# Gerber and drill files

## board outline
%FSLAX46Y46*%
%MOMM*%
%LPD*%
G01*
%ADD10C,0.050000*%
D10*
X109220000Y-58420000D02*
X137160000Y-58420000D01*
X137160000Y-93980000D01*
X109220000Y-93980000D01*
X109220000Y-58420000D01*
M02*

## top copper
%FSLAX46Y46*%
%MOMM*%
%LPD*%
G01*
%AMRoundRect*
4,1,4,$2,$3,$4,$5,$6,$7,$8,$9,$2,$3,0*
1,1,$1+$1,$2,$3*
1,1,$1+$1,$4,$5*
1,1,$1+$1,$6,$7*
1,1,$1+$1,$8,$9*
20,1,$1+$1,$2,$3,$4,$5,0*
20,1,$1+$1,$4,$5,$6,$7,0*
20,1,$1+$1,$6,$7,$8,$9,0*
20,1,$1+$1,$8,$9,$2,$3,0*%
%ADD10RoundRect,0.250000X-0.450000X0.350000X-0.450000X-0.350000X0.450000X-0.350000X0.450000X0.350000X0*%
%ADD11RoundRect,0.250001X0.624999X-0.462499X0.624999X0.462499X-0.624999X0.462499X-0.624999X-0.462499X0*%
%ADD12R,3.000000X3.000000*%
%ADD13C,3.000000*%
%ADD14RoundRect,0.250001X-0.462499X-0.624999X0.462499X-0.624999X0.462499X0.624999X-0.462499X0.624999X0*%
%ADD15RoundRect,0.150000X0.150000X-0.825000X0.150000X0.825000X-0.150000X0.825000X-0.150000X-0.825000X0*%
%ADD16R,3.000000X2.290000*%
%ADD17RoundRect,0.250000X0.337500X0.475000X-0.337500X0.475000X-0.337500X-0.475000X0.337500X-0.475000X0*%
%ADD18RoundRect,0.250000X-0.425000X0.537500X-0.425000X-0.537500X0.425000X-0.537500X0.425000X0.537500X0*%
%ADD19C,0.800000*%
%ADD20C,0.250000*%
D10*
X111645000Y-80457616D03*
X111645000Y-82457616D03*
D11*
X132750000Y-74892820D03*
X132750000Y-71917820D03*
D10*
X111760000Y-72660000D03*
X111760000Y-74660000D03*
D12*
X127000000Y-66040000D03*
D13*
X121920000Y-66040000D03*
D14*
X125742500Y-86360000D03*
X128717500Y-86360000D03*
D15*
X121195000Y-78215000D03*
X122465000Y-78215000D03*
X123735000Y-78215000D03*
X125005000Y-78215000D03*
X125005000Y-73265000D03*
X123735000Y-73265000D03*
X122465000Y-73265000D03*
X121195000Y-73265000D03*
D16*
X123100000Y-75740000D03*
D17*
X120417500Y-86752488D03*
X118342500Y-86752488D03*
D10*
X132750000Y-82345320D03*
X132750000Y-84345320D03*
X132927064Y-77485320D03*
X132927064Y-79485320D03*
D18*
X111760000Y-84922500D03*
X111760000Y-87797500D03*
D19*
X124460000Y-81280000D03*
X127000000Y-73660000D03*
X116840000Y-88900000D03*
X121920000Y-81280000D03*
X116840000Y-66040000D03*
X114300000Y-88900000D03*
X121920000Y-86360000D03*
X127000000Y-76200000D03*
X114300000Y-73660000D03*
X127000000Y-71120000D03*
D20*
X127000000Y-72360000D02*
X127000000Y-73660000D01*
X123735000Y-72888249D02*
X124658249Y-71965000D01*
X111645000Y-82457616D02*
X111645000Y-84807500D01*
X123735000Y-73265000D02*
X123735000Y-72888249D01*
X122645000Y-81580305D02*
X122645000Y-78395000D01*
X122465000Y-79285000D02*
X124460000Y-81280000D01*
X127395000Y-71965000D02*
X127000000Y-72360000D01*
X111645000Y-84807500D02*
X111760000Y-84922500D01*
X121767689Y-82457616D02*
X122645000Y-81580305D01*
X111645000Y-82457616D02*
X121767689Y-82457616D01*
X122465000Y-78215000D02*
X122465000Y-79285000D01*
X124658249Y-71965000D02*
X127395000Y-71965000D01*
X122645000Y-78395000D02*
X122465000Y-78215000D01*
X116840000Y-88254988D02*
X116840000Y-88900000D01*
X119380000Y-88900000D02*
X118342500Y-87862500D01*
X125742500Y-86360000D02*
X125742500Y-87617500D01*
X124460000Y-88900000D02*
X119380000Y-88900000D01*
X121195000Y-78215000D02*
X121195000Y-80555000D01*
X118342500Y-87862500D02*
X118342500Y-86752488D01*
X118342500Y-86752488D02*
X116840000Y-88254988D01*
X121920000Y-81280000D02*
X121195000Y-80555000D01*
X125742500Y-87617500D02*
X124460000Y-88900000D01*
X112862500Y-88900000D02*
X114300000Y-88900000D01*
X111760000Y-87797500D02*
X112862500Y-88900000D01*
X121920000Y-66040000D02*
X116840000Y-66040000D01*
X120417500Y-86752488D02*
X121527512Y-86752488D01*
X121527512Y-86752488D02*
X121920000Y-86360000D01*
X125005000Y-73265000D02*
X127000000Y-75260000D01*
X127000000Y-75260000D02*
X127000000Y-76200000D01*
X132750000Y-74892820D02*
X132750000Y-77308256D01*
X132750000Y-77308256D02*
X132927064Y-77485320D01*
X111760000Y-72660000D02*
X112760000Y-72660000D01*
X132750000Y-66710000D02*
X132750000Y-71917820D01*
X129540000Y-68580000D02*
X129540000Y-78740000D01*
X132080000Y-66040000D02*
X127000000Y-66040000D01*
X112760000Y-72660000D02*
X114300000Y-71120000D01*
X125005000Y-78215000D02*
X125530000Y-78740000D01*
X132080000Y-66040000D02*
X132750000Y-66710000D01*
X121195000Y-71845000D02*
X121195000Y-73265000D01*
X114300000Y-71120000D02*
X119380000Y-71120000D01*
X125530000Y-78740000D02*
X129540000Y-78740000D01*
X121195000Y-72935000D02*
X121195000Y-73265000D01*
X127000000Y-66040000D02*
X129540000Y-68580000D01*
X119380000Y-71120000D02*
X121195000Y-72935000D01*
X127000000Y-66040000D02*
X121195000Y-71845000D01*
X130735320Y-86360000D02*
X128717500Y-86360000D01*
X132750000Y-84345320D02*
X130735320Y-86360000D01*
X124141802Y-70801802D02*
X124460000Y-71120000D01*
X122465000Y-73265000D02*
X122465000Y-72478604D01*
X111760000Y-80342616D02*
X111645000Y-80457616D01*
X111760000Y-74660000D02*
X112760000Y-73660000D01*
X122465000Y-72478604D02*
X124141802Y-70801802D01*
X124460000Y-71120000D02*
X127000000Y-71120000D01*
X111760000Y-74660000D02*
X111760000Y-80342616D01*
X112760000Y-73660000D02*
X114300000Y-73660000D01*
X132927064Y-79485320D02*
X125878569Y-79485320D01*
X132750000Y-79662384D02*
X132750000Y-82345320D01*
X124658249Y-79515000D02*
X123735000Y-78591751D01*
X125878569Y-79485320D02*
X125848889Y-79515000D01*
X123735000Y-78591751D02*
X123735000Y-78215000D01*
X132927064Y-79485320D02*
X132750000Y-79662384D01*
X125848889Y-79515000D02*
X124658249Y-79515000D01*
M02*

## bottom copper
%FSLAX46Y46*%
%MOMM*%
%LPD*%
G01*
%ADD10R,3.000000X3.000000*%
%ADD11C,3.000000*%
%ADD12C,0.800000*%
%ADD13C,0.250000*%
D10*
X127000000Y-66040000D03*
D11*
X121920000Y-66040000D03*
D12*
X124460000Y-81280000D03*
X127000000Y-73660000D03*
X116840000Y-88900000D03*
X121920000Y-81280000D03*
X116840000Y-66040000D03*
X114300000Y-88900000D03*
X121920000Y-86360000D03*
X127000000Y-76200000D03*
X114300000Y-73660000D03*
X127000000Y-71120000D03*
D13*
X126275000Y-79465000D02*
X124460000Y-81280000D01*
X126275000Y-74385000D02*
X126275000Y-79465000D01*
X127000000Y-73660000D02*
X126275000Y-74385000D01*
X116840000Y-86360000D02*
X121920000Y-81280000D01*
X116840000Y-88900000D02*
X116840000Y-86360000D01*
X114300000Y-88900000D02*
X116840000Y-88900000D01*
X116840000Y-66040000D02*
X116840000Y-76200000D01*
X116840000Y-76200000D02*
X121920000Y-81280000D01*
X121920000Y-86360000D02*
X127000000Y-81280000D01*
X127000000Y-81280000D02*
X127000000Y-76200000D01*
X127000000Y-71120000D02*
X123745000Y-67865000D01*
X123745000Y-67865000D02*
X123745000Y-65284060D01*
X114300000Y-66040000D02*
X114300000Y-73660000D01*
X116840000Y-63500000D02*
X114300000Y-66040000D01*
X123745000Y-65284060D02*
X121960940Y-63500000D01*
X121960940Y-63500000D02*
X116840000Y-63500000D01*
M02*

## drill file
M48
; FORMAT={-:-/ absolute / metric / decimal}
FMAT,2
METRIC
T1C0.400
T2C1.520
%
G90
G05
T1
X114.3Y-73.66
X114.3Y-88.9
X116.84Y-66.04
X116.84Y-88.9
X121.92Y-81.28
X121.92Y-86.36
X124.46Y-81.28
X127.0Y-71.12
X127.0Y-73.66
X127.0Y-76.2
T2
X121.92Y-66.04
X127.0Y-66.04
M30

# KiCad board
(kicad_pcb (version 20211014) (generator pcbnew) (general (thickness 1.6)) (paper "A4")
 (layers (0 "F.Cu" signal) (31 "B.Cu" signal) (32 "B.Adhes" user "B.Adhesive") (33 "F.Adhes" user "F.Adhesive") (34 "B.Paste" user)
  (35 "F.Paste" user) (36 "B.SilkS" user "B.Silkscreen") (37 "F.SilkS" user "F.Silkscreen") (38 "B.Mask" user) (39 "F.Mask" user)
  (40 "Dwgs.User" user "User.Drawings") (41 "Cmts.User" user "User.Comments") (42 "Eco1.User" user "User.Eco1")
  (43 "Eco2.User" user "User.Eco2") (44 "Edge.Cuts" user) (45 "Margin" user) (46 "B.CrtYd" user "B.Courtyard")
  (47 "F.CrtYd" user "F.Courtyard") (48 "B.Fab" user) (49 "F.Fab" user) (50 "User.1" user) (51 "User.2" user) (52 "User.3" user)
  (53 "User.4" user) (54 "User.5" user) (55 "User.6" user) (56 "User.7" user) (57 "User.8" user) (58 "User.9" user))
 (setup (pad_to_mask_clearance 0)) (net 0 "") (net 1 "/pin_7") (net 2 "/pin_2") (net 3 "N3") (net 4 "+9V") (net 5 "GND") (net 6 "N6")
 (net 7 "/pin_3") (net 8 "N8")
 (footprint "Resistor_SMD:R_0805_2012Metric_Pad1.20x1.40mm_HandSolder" (layer "F.Cu") (at 111.645 81.457616 -90)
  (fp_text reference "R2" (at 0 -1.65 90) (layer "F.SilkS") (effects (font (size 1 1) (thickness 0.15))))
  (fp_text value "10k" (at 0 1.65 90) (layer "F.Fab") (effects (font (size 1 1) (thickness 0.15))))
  (pad "1" smd roundrect (at -1 0 270) (size 1.2 1.4) (layers "F.Cu" "F.Paste" "F.Mask") (roundrect_rratio 0.208333) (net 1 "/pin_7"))
  (pad "2" smd roundrect (at 1 0 270) (size 1.2 1.4) (layers "F.Cu" "F.Paste" "F.Mask") (roundrect_rratio 0.208333) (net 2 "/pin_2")))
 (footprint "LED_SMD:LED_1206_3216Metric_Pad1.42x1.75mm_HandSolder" (layer "F.Cu") (at 132.75 73.40532 90)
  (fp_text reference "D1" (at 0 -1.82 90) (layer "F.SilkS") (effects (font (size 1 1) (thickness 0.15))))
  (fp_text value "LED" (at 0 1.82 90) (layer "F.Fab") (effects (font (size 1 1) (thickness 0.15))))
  (pad "1" smd roundrect (at -1.4875 0 90) (size 1.425 1.75) (layers "F.Cu" "F.Paste" "F.Mask") (roundrect_rratio 0.175439) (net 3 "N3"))
  (pad "2" smd roundrect (at 1.4875 0 90) (size 1.425 1.75) (layers "F.Cu" "F.Paste" "F.Mask") (roundrect_rratio 0.175439) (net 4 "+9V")))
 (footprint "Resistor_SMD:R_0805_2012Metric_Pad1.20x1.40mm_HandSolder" (layer "F.Cu") (at 111.76 73.66 -90)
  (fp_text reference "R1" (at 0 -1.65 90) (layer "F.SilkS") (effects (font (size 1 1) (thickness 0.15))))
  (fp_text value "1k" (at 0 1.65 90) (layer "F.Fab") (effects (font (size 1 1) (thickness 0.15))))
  (pad "1" smd roundrect (at -1 0 270) (size 1.2 1.4) (layers "F.Cu" "F.Paste" "F.Mask") (roundrect_rratio 0.208333) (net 4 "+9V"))
  (pad "2" smd roundrect (at 1 0 270) (size 1.2 1.4) (layers "F.Cu" "F.Paste" "F.Mask") (roundrect_rratio 0.208333) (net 1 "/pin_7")))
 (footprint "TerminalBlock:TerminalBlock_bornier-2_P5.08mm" (layer "F.Cu") (at 127 66.04 180)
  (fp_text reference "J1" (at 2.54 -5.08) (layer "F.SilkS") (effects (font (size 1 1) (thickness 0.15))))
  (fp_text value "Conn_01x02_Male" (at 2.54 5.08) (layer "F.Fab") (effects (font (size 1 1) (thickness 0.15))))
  (pad "1" thru_hole rect (at 0 0 180) (size 3 3) (drill 1.52) (layers *.Cu *.Mask) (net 4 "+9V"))
  (pad "2" thru_hole circle (at 5.08 0 180) (size 3 3) (drill 1.52) (layers *.Cu *.Mask) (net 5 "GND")))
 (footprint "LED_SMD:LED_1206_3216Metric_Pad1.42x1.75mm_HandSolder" (layer "F.Cu") (at 127.23 86.36)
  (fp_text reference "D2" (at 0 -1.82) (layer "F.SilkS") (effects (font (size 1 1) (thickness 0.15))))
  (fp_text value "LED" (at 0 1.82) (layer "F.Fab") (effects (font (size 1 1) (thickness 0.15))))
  (pad "1" smd roundrect (at -1.4875 0) (size 1.425 1.75) (layers "F.Cu" "F.Paste" "F.Mask") (roundrect_rratio 0.175439) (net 5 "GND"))
  (pad "2" smd roundrect (at 1.4875 0) (size 1.425 1.75) (layers "F.Cu" "F.Paste" "F.Mask") (roundrect_rratio 0.175439) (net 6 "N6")))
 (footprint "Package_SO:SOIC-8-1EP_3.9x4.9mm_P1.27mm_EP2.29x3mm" (layer "F.Cu") (at 123.1 75.74 90)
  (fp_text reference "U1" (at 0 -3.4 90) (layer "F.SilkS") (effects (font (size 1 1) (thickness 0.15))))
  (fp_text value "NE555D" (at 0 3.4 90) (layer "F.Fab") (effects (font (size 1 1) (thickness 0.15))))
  (pad "" smd roundrect (at 0.57 -0.75 90) (size 0.92 1.21) (layers "F.Paste") (roundrect_rratio 0.25))
  (pad "" smd roundrect (at 0.57 0.75 90) (size 0.92 1.21) (layers "F.Paste") (roundrect_rratio 0.25))
  (pad "" smd roundrect (at -0.57 0.75 90) (size 0.92 1.21) (layers "F.Paste") (roundrect_rratio 0.25))
  (pad "" smd roundrect (at -0.57 -0.75 90) (size 0.92 1.21) (layers "F.Paste") (roundrect_rratio 0.25))
  (pad "1" smd roundrect (at -2.475 -1.905 90) (size 1.95 0.6) (layers "F.Cu" "F.Paste" "F.Mask") (roundrect_rratio 0.25) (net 5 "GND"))
  (pad "2" smd roundrect (at -2.475 -0.635 90) (size 1.95 0.6) (layers "F.Cu" "F.Paste" "F.Mask") (roundrect_rratio 0.25) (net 2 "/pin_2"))
  (pad "3" smd roundrect (at -2.475 0.635 90) (size 1.95 0.6) (layers "F.Cu" "F.Paste" "F.Mask") (roundrect_rratio 0.25) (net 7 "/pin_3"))
  (pad "4" smd roundrect (at -2.475 1.905 90) (size 1.95 0.6) (layers "F.Cu" "F.Paste" "F.Mask") (roundrect_rratio 0.25) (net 4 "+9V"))
  (pad "5" smd roundrect (at 2.475 1.905 90) (size 1.95 0.6) (layers "F.Cu" "F.Paste" "F.Mask") (roundrect_rratio 0.25) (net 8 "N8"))
  (pad "6" smd roundrect (at 2.475 0.635 90) (size 1.95 0.6) (layers "F.Cu" "F.Paste" "F.Mask") (roundrect_rratio 0.25) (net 2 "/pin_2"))
  (pad "7" smd roundrect (at 2.475 -0.635 90) (size 1.95 0.6) (layers "F.Cu" "F.Paste" "F.Mask") (roundrect_rratio 0.25) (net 1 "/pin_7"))
  (pad "8" smd roundrect (at 2.475 -1.905 90) (size 1.95 0.6) (layers "F.Cu" "F.Paste" "F.Mask") (roundrect_rratio 0.25) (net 4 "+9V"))
  (pad "9" smd rect (at 0 0 90) (size 2.29 3) (layers "F.Cu" "F.Mask")))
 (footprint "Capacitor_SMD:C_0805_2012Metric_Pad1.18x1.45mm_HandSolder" (layer "F.Cu") (at 119.38 86.752488 180)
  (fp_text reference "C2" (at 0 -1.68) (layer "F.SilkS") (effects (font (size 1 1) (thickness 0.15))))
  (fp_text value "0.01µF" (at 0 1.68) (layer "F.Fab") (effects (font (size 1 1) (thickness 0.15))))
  (pad "1" smd roundrect (at -1.0375 0 180) (size 1.175 1.45) (layers "F.Cu" "F.Paste" "F.Mask") (roundrect_rratio 0.212766) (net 8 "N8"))
  (pad "2" smd roundrect (at 1.0375 0 180) (size 1.175 1.45) (layers "F.Cu" "F.Paste" "F.Mask") (roundrect_rratio 0.212766) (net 5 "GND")))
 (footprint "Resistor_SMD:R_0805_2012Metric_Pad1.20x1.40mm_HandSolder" (layer "F.Cu") (at 132.75 83.34532 -90)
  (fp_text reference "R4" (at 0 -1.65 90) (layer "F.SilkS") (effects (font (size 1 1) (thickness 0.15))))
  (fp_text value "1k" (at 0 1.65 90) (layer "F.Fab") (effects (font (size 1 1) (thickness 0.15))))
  (pad "1" smd roundrect (at -1 0 270) (size 1.2 1.4) (layers "F.Cu" "F.Paste" "F.Mask") (roundrect_rratio 0.208333) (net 7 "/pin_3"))
  (pad "2" smd roundrect (at 1 0 270) (size 1.2 1.4) (layers "F.Cu" "F.Paste" "F.Mask") (roundrect_rratio 0.208333) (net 6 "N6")))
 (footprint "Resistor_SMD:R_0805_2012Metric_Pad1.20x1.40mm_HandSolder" (layer "F.Cu") (at 132.927064 78.48532 -90)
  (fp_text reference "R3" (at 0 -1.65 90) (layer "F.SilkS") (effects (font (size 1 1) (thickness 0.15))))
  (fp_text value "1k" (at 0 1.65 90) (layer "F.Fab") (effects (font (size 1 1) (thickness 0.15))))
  (pad "1" smd roundrect (at -1 0 270) (size 1.2 1.4) (layers "F.Cu" "F.Paste" "F.Mask") (roundrect_rratio 0.208333) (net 3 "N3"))
  (pad "2" smd roundrect (at 1 0 270) (size 1.2 1.4) (layers "F.Cu" "F.Paste" "F.Mask") (roundrect_rratio 0.208333) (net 7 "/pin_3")))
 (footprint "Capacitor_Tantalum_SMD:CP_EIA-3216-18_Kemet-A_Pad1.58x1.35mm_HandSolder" (layer "F.Cu") (at 111.76 86.36 -90)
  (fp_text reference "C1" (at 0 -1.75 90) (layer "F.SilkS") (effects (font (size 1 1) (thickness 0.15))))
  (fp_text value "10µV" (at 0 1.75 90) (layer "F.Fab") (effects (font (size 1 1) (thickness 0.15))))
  (pad "1" smd roundrect (at -1.4375 0 270) (size 1.575 1.35) (layers "F.Cu" "F.Paste" "F.Mask") (roundrect_rratio 0.185185)
   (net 2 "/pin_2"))
  (pad "2" smd roundrect (at 1.4375 0 270) (size 1.575 1.35) (layers "F.Cu" "F.Paste" "F.Mask") (roundrect_rratio 0.185185) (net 5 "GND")))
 (gr_rect (start 109.22 58.42) (end 137.16 93.98) (layer "Edge.Cuts") (width 0.05) (fill none))
 (segment (start 127 72.36) (end 127 73.66) (width 0.25) (layer "F.Cu") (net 2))
 (segment (start 123.735 72.888249) (end 124.658249 71.965) (width 0.25) (layer "F.Cu") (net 2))
 (segment (start 111.645 82.457616) (end 111.645 84.8075) (width 0.25) (layer "F.Cu") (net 2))
 (segment (start 123.735 73.265) (end 123.735 72.888249) (width 0.25) (layer "F.Cu") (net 2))
 (segment (start 122.645 81.580305) (end 122.645 78.395) (width 0.25) (layer "F.Cu") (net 2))
 (segment (start 122.465 79.285) (end 124.46 81.28) (width 0.25) (layer "F.Cu") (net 2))
 (segment (start 127.395 71.965) (end 127 72.36) (width 0.25) (layer "F.Cu") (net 2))
 (segment (start 111.645 84.8075) (end 111.76 84.9225) (width 0.25) (layer "F.Cu") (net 2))
 (segment (start 121.767689 82.457616) (end 122.645 81.580305) (width 0.25) (layer "F.Cu") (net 2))
 (segment (start 111.645 82.457616) (end 121.767689 82.457616) (width 0.25) (layer "F.Cu") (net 2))
 (segment (start 122.465 78.215) (end 122.465 79.285) (width 0.25) (layer "F.Cu") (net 2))
 (segment (start 124.658249 71.965) (end 127.395 71.965) (width 0.25) (layer "F.Cu") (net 2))
 (segment (start 122.645 78.395) (end 122.465 78.215) (width 0.25) (layer "F.Cu") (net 2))
 (via (at 124.46 81.28) (size 0.8) (drill 0.4) (layers "F.Cu" "B.Cu") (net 2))
 (via (at 127 73.66) (size 0.8) (drill 0.4) (layers "F.Cu" "B.Cu") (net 2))
 (segment (start 126.275 79.465) (end 124.46 81.28) (width 0.25) (layer "B.Cu") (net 2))
 (segment (start 126.275 74.385) (end 126.275 79.465) (width 0.25) (layer "B.Cu") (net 2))
 (segment (start 127 73.66) (end 126.275 74.385) (width 0.25) (layer "B.Cu") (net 2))
 (segment (start 116.84 88.254988) (end 116.84 88.9) (width 0.25) (layer "F.Cu") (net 5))
 (segment (start 119.38 88.9) (end 118.3425 87.8625) (width 0.25) (layer "F.Cu") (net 5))
 (segment (start 125.7425 86.36) (end 125.7425 87.6175) (width 0.25) (layer "F.Cu") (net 5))
 (segment (start 124.46 88.9) (end 119.38 88.9) (width 0.25) (layer "F.Cu") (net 5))
 (segment (start 121.195 78.215) (end 121.195 80.555) (width 0.25) (layer "F.Cu") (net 5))
 (segment (start 118.3425 87.8625) (end 118.3425 86.752488) (width 0.25) (layer "F.Cu") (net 5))
 (segment (start 118.3425 86.752488) (end 116.84 88.254988) (width 0.25) (layer "F.Cu") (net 5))
 (segment (start 121.92 81.28) (end 121.195 80.555) (width 0.25) (layer "F.Cu") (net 5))
 (segment (start 125.7425 87.6175) (end 124.46 88.9) (width 0.25) (layer "F.Cu") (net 5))
 (segment (start 112.8625 88.9) (end 114.3 88.9) (width 0.25) (layer "F.Cu") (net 5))
 (segment (start 111.76 87.7975) (end 112.8625 88.9) (width 0.25) (layer "F.Cu") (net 5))
 (segment (start 121.92 66.04) (end 116.84 66.04) (width 0.25) (layer "F.Cu") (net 5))
 (via (at 116.84 88.9) (size 0.8) (drill 0.4) (layers "F.Cu" "B.Cu") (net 5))
 (via (at 121.92 81.28) (size 0.8) (drill 0.4) (layers "F.Cu" "B.Cu") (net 5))
 (via (at 116.84 66.04) (size 0.8) (drill 0.4) (layers "F.Cu" "B.Cu") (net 5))
 (via (at 114.3 88.9) (size 0.8) (drill 0.4) (layers "F.Cu" "B.Cu") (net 5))
 (segment (start 116.84 86.36) (end 121.92 81.28) (width 0.25) (layer "B.Cu") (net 5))
 (segment (start 116.84 88.9) (end 116.84 86.36) (width 0.25) (layer "B.Cu") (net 5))
 (segment (start 114.3 88.9) (end 116.84 88.9) (width 0.25) (layer "B.Cu") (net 5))
 (segment (start 116.84 66.04) (end 116.84 76.2) (width 0.25) (layer "B.Cu") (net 5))
 (segment (start 116.84 76.2) (end 121.92 81.28) (width 0.25) (layer "B.Cu") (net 5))
 (segment (start 120.4175 86.752488) (end 121.527512 86.752488) (width 0.25) (layer "F.Cu") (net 8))
 (segment (start 121.527512 86.752488) (end 121.92 86.36) (width 0.25) (layer "F.Cu") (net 8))
 (segment (start 125.005 73.265) (end 127 75.26) (width 0.25) (layer "F.Cu") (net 8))
 (segment (start 127 75.26) (end 127 76.2) (width 0.25) (layer "F.Cu") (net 8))
 (via (at 121.92 86.36) (size 0.8) (drill 0.4) (layers "F.Cu" "B.Cu") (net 8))
 (via (at 127 76.2) (size 0.8) (drill 0.4) (layers "F.Cu" "B.Cu") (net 8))
 (segment (start 121.92 86.36) (end 127 81.28) (width 0.25) (layer "B.Cu") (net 8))
 (segment (start 127 81.28) (end 127 76.2) (width 0.25) (layer "B.Cu") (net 8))
 (segment (start 132.75 74.89282) (end 132.75 77.308256) (width 0.25) (layer "F.Cu") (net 3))
 (segment (start 132.75 77.308256) (end 132.927064 77.48532) (width 0.25) (layer "F.Cu") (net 3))
 (segment (start 111.76 72.66) (end 112.76 72.66) (width 0.25) (layer "F.Cu") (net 4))
 (segment (start 132.75 66.71) (end 132.75 71.91782) (width 0.25) (layer "F.Cu") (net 4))
 (segment (start 129.54 68.58) (end 129.54 78.74) (width 0.25) (layer "F.Cu") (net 4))
 (segment (start 132.08 66.04) (end 127 66.04) (width 0.25) (layer "F.Cu") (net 4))
 (segment (start 112.76 72.66) (end 114.3 71.12) (width 0.25) (layer "F.Cu") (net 4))
 (segment (start 125.005 78.215) (end 125.53 78.74) (width 0.25) (layer "F.Cu") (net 4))
 (segment (start 132.08 66.04) (end 132.75 66.71) (width 0.25) (layer "F.Cu") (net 4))
 (segment (start 121.195 71.845) (end 121.195 73.265) (width 0.25) (layer "F.Cu") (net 4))
 (segment (start 114.3 71.12) (end 119.38 71.12) (width 0.25) (layer "F.Cu") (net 4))
 (segment (start 125.53 78.74) (end 129.54 78.74) (width 0.25) (layer "F.Cu") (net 4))
 (segment (start 121.195 72.935) (end 121.195 73.265) (width 0.25) (layer "F.Cu") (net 4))
 (segment (start 127 66.04) (end 129.54 68.58) (width 0.25) (layer "F.Cu") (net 4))
 (segment (start 119.38 71.12) (end 121.195 72.935) (width 0.25) (layer "F.Cu") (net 4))
 (segment (start 127 66.04) (end 121.195 71.845) (width 0.25) (layer "F.Cu") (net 4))
 (segment (start 130.73532 86.36) (end 128.7175 86.36) (width 0.25) (layer "F.Cu") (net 6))
 (segment (start 132.75 84.34532) (end 130.73532 86.36) (width 0.25) (layer "F.Cu") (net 6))
 (segment (start 124.141802 70.801802) (end 124.46 71.12) (width 0.25) (layer "F.Cu") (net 1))
 (segment (start 122.465 73.265) (end 122.465 72.478604) (width 0.25) (layer "F.Cu") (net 1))
 (segment (start 111.76 80.342616) (end 111.645 80.457616) (width 0.25) (layer "F.Cu") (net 1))
 (segment (start 111.76 74.66) (end 112.76 73.66) (width 0.25) (layer "F.Cu") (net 1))
 (segment (start 122.465 72.478604) (end 124.141802 70.801802) (width 0.25) (layer "F.Cu") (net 1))
 (segment (start 124.46 71.12) (end 127 71.12) (width 0.25) (layer "F.Cu") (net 1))
 (segment (start 111.76 74.66) (end 111.76 80.342616) (width 0.25) (layer "F.Cu") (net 1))
 (segment (start 112.76 73.66) (end 114.3 73.66) (width 0.25) (layer "F.Cu") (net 1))
 (via (at 114.3 73.66) (size 0.8) (drill 0.4) (layers "F.Cu" "B.Cu") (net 1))
 (via (at 127 71.12) (size 0.8) (drill 0.4) (layers "F.Cu" "B.Cu") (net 1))
 (segment (start 127 71.12) (end 123.745 67.865) (width 0.25) (layer "B.Cu") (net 1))
 (segment (start 123.745 67.865) (end 123.745 65.28406) (width 0.25) (layer "B.Cu") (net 1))
 (segment (start 114.3 66.04) (end 114.3 73.66) (width 0.25) (layer "B.Cu") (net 1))
 (segment (start 116.84 63.5) (end 114.3 66.04) (width 0.25) (layer "B.Cu") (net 1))
 (segment (start 123.745 65.28406) (end 121.96094 63.5) (width 0.25) (layer "B.Cu") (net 1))
 (segment (start 121.96094 63.5) (end 116.84 63.5) (width 0.25) (layer "B.Cu") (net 1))
 (segment (start 132.927064 79.48532) (end 125.878569 79.48532) (width 0.25) (layer "F.Cu") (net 7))
 (segment (start 132.75 79.662384) (end 132.75 82.34532) (width 0.25) (layer "F.Cu") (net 7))
 (segment (start 124.658249 79.515) (end 123.735 78.591751) (width 0.25) (layer "F.Cu") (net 7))
 (segment (start 125.878569 79.48532) (end 125.848889 79.515) (width 0.25) (layer "F.Cu") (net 7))
 (segment (start 123.735 78.591751) (end 123.735 78.215) (width 0.25) (layer "F.Cu") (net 7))
 (segment (start 132.927064 79.48532) (end 132.75 79.662384) (width 0.25) (layer "F.Cu") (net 7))
 (segment (start 125.848889 79.515) (end 124.658249 79.515) (width 0.25) (layer "F.Cu") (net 7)))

